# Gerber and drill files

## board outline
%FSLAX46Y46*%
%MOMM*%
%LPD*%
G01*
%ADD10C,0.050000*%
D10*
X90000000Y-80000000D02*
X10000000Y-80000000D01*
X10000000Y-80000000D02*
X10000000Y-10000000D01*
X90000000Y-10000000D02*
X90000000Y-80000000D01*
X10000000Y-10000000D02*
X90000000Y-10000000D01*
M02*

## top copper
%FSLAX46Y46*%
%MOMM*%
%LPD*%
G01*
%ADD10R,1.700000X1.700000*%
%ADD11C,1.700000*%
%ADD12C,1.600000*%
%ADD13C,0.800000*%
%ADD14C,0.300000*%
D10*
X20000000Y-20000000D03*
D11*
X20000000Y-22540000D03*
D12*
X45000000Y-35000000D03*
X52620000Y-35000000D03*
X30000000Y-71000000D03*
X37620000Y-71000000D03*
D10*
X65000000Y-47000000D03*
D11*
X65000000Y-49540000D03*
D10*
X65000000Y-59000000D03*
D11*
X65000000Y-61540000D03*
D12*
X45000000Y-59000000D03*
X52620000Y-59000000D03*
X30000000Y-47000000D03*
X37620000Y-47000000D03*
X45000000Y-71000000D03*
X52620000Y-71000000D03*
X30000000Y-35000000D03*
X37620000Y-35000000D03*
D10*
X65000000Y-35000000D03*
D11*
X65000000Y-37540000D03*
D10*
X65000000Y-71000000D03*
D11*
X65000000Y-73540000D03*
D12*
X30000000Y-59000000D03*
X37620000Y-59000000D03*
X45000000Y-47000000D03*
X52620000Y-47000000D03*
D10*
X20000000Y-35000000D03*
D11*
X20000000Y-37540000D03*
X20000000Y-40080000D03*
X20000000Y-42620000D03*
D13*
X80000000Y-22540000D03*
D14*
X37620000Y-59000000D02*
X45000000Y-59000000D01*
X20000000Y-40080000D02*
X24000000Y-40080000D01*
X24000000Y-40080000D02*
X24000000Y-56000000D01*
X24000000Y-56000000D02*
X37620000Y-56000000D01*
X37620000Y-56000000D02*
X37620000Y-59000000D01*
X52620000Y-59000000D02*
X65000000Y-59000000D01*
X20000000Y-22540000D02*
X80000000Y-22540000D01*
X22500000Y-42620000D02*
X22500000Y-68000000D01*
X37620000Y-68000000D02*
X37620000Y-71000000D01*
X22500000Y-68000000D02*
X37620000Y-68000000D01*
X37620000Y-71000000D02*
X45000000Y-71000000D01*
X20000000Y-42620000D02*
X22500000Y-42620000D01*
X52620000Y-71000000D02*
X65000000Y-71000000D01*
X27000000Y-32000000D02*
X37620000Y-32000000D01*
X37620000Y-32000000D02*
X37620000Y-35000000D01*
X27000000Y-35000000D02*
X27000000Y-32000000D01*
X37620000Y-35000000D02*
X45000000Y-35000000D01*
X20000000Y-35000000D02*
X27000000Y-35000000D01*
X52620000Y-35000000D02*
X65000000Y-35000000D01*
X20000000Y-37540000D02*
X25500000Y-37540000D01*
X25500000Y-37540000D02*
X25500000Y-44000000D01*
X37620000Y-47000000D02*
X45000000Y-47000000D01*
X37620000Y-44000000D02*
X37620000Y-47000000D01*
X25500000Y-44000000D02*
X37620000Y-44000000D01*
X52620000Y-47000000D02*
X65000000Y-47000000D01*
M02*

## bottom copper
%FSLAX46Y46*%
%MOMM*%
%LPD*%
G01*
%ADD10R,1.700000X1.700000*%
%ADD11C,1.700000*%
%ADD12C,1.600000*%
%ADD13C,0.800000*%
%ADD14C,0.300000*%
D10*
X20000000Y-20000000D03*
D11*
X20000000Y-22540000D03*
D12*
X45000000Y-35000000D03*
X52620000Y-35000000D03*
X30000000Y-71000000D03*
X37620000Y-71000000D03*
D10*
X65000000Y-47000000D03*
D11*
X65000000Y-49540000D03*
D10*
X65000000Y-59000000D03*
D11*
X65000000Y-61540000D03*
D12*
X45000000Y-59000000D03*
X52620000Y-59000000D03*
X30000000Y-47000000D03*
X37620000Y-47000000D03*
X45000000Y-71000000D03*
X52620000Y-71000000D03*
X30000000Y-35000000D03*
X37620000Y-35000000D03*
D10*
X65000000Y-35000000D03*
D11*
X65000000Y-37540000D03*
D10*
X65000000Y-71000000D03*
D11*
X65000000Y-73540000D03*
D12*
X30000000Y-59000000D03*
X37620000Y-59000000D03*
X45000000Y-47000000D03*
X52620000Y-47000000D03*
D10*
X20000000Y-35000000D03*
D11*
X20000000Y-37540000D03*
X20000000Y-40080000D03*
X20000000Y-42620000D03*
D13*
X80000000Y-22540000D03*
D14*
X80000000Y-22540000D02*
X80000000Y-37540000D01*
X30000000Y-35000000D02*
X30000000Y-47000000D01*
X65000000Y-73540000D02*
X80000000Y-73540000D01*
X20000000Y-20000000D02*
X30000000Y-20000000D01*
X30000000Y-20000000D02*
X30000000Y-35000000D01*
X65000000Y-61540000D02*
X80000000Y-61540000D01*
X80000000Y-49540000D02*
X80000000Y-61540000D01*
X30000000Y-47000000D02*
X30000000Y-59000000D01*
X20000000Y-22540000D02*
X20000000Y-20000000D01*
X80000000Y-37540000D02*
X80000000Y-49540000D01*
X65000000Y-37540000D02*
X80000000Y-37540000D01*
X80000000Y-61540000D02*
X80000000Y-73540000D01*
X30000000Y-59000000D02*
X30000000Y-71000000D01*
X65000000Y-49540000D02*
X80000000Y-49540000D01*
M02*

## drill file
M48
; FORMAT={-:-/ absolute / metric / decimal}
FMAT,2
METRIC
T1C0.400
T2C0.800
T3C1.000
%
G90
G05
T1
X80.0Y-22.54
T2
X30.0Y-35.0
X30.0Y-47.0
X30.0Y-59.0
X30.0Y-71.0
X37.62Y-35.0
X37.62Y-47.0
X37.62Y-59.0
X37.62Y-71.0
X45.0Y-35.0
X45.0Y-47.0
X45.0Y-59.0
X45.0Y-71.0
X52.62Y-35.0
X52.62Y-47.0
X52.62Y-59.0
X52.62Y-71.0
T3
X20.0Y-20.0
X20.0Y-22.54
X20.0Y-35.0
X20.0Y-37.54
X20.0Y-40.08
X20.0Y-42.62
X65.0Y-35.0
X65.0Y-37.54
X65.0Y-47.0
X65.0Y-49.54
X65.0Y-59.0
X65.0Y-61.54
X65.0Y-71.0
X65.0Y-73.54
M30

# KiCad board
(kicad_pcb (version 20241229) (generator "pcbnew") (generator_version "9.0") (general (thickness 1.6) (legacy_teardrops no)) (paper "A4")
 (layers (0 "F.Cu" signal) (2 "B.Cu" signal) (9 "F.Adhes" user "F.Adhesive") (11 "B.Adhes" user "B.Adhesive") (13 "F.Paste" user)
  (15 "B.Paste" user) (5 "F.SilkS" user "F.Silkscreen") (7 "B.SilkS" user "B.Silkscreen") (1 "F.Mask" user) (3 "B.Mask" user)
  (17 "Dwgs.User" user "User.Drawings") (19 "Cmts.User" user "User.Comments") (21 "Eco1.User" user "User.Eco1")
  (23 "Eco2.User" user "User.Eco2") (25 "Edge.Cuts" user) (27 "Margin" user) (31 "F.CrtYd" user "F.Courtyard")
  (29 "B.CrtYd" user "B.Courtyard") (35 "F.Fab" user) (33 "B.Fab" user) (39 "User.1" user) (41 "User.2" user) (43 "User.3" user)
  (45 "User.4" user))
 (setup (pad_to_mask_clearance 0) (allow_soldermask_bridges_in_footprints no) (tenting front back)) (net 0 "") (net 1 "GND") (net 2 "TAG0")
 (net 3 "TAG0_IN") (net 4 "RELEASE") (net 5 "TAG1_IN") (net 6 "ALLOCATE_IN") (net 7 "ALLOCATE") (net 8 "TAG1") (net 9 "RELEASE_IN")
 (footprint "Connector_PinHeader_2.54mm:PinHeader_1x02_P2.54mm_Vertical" (layer "F.Cu") (at 20 20)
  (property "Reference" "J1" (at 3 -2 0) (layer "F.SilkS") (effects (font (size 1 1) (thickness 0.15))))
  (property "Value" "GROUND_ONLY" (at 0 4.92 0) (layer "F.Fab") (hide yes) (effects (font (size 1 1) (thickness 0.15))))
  (pad "1" thru_hole rect (at 0 0) (size 1.7 1.7) (drill 1) (layers "*.Cu" "*.Mask") (remove_unused_layers no) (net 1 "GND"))
  (pad "2" thru_hole circle (at 0 2.54) (size 1.7 1.7) (drill 1) (layers "*.Cu" "*.Mask") (remove_unused_layers no) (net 1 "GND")))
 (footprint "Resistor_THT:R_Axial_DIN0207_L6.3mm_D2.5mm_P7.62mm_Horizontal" (layer "F.Cu") (at 45 35)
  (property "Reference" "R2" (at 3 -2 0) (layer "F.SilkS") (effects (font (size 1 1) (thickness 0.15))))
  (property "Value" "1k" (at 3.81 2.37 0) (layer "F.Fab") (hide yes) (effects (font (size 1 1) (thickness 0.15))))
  (pad "1" thru_hole circle (at 0 0) (size 1.6 1.6) (drill 0.8) (layers "*.Cu" "*.Mask") (remove_unused_layers no) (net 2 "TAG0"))
  (pad "2" thru_hole circle (at 7.62 0) (size 1.6 1.6) (drill 0.8) (layers "*.Cu" "*.Mask") (remove_unused_layers no) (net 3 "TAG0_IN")))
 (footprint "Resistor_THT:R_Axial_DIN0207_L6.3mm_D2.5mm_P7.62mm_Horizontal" (layer "F.Cu") (at 30 71)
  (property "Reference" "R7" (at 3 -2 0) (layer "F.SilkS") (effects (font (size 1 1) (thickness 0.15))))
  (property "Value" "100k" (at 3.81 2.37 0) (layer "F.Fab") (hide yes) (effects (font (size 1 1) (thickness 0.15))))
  (pad "1" thru_hole circle (at 0 0) (size 1.6 1.6) (drill 0.8) (layers "*.Cu" "*.Mask") (remove_unused_layers no) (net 1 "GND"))
  (pad "2" thru_hole circle (at 7.62 0) (size 1.6 1.6) (drill 0.8) (layers "*.Cu" "*.Mask") (remove_unused_layers no) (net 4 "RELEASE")))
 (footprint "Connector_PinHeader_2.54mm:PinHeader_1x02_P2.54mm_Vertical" (layer "F.Cu") (at 65 47)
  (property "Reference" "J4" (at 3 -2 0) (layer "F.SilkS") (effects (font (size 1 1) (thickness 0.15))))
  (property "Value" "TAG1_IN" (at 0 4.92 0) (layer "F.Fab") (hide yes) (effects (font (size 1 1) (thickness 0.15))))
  (pad "1" thru_hole rect (at 0 0) (size 1.7 1.7) (drill 1) (layers "*.Cu" "*.Mask") (remove_unused_layers no) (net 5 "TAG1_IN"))
  (pad "2" thru_hole circle (at 0 2.54) (size 1.7 1.7) (drill 1) (layers "*.Cu" "*.Mask") (remove_unused_layers no) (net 1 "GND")))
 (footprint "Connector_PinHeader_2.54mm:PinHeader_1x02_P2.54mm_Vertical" (layer "F.Cu") (at 65 59)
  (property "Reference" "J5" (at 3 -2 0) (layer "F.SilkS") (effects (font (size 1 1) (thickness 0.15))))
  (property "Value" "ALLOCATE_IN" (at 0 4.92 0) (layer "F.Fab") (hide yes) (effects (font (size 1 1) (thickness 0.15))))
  (pad "1" thru_hole rect (at 0 0) (size 1.7 1.7) (drill 1) (layers "*.Cu" "*.Mask") (remove_unused_layers no) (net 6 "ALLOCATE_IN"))
  (pad "2" thru_hole circle (at 0 2.54) (size 1.7 1.7) (drill 1) (layers "*.Cu" "*.Mask") (remove_unused_layers no) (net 1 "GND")))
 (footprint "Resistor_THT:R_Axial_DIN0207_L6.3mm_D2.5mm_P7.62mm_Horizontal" (layer "F.Cu") (at 45 59)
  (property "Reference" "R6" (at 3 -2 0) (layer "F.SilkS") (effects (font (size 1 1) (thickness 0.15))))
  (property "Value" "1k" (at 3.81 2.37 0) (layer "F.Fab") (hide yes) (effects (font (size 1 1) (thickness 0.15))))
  (pad "1" thru_hole circle (at 0 0) (size 1.6 1.6) (drill 0.8) (layers "*.Cu" "*.Mask") (remove_unused_layers no) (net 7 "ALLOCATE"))
  (pad "2" thru_hole circle (at 7.62 0) (size 1.6 1.6) (drill 0.8) (layers "*.Cu" "*.Mask") (remove_unused_layers no) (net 6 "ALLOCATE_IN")))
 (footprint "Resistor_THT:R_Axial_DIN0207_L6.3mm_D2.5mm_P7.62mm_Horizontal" (layer "F.Cu") (at 30 47)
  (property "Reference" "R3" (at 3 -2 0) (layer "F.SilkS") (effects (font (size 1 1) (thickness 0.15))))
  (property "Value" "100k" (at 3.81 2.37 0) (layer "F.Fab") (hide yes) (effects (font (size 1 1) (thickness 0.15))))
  (pad "1" thru_hole circle (at 0 0) (size 1.6 1.6) (drill 0.8) (layers "*.Cu" "*.Mask") (remove_unused_layers no) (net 1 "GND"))
  (pad "2" thru_hole circle (at 7.62 0) (size 1.6 1.6) (drill 0.8) (layers "*.Cu" "*.Mask") (remove_unused_layers no) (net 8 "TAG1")))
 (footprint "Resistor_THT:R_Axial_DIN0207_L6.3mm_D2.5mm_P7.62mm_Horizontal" (layer "F.Cu") (at 45 71)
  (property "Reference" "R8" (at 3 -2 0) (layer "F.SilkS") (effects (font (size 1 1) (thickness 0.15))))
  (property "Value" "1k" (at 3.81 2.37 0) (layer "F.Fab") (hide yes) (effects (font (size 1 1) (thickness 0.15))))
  (pad "1" thru_hole circle (at 0 0) (size 1.6 1.6) (drill 0.8) (layers "*.Cu" "*.Mask") (remove_unused_layers no) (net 4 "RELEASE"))
  (pad "2" thru_hole circle (at 7.62 0) (size 1.6 1.6) (drill 0.8) (layers "*.Cu" "*.Mask") (remove_unused_layers no) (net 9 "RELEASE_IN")))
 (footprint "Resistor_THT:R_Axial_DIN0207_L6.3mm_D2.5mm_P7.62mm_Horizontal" (layer "F.Cu") (at 30 35)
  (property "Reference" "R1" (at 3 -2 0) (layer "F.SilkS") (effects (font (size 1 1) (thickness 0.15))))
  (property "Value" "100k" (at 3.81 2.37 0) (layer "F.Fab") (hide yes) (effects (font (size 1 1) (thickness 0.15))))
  (pad "1" thru_hole circle (at 0 0) (size 1.6 1.6) (drill 0.8) (layers "*.Cu" "*.Mask") (remove_unused_layers no) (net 1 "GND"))
  (pad "2" thru_hole circle (at 7.62 0) (size 1.6 1.6) (drill 0.8) (layers "*.Cu" "*.Mask") (remove_unused_layers no) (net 2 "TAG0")))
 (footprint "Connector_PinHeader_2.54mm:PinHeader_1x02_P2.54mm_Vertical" (layer "F.Cu") (at 65 35)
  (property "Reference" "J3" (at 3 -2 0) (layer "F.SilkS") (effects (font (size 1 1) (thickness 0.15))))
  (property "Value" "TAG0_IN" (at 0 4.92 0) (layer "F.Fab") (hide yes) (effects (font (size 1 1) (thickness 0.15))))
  (pad "1" thru_hole rect (at 0 0) (size 1.7 1.7) (drill 1) (layers "*.Cu" "*.Mask") (remove_unused_layers no) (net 3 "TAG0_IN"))
  (pad "2" thru_hole circle (at 0 2.54) (size 1.7 1.7) (drill 1) (layers "*.Cu" "*.Mask") (remove_unused_layers no) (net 1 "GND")))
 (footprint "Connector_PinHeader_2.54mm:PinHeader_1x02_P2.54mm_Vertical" (layer "F.Cu") (at 65 71)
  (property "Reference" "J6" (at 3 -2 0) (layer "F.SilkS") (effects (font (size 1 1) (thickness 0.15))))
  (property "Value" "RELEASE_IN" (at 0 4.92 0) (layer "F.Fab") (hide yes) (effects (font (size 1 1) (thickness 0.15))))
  (pad "1" thru_hole rect (at 0 0) (size 1.7 1.7) (drill 1) (layers "*.Cu" "*.Mask") (remove_unused_layers no) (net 9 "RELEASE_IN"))
  (pad "2" thru_hole circle (at 0 2.54) (size 1.7 1.7) (drill 1) (layers "*.Cu" "*.Mask") (remove_unused_layers no) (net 1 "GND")))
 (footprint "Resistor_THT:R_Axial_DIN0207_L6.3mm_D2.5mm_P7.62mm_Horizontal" (layer "F.Cu") (at 30 59)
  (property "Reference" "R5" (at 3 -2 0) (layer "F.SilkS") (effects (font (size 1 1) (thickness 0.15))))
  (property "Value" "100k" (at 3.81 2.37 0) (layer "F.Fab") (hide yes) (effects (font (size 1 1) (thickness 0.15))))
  (pad "1" thru_hole circle (at 0 0) (size 1.6 1.6) (drill 0.8) (layers "*.Cu" "*.Mask") (remove_unused_layers no) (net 1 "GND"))
  (pad "2" thru_hole circle (at 7.62 0) (size 1.6 1.6) (drill 0.8) (layers "*.Cu" "*.Mask") (remove_unused_layers no) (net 7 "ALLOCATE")))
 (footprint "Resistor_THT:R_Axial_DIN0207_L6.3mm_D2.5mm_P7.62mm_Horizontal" (layer "F.Cu") (at 45 47)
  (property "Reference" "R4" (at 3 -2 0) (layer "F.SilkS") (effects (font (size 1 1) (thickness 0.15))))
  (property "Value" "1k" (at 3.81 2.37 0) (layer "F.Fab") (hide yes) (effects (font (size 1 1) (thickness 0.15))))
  (pad "1" thru_hole circle (at 0 0) (size 1.6 1.6) (drill 0.8) (layers "*.Cu" "*.Mask") (remove_unused_layers no) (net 8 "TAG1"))
  (pad "2" thru_hole circle (at 7.62 0) (size 1.6 1.6) (drill 0.8) (layers "*.Cu" "*.Mask") (remove_unused_layers no) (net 5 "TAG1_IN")))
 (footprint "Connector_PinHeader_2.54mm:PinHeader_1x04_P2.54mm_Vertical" (layer "F.Cu") (at 20 35)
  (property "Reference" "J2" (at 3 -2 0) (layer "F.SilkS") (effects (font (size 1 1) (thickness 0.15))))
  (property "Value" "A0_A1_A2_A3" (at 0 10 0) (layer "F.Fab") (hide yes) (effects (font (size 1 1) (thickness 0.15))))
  (pad "1" thru_hole rect (at 0 0) (size 1.7 1.7) (drill 1) (layers "*.Cu" "*.Mask") (remove_unused_layers no) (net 2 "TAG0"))
  (pad "2" thru_hole circle (at 0 2.54) (size 1.7 1.7) (drill 1) (layers "*.Cu" "*.Mask") (remove_unused_layers no) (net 8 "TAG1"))
  (pad "3" thru_hole circle (at 0 5.08) (size 1.7 1.7) (drill 1) (layers "*.Cu" "*.Mask") (remove_unused_layers no) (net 7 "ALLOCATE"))
  (pad "4" thru_hole circle (at 0 7.62) (size 1.7 1.7) (drill 1) (layers "*.Cu" "*.Mask") (remove_unused_layers no) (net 4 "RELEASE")))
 (gr_line (start 90 80) (end 10 80) (stroke (width 0.05) (type default)) (layer "Edge.Cuts"))
 (gr_line (start 10 80) (end 10 10) (stroke (width 0.05) (type default)) (layer "Edge.Cuts"))
 (gr_line (start 90 10) (end 90 80) (stroke (width 0.05) (type default)) (layer "Edge.Cuts"))
 (gr_line (start 10 10) (end 90 10) (stroke (width 0.05) (type default)) (layer "Edge.Cuts"))
 (segment (start 37.62 59) (end 45 59) (width 0.3) (layer "F.Cu") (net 7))
 (segment (start 20 40.08) (end 24 40.08) (width 0.3) (layer "F.Cu") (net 7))
 (segment (start 24 40.08) (end 24 56) (width 0.3) (layer "F.Cu") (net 7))
 (segment (start 24 56) (end 37.62 56) (width 0.3) (layer "F.Cu") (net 7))
 (segment (start 37.62 56) (end 37.62 59) (width 0.3) (layer "F.Cu") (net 7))
 (segment (start 52.62 59) (end 65 59) (width 0.3) (layer "F.Cu") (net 6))
 (segment (start 20 22.54) (end 80 22.54) (width 0.3) (layer "F.Cu") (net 1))
 (via (at 80 22.54) (size 0.8) (drill 0.4) (layers "F.Cu" "B.Cu") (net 1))
 (segment (start 80 22.54) (end 80 37.54) (width 0.3) (layer "B.Cu") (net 1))
 (segment (start 30 35) (end 30 47) (width 0.3) (layer "B.Cu") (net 1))
 (segment (start 65 73.54) (end 80 73.54) (width 0.3) (layer "B.Cu") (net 1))
 (segment (start 20 20) (end 30 20) (width 0.3) (layer "B.Cu") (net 1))
 (segment (start 30 20) (end 30 35) (width 0.3) (layer "B.Cu") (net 1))
 (segment (start 65 61.54) (end 80 61.54) (width 0.3) (layer "B.Cu") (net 1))
 (segment (start 80 49.54) (end 80 61.54) (width 0.3) (layer "B.Cu") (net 1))
 (segment (start 30 47) (end 30 59) (width 0.3) (layer "B.Cu") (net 1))
 (segment (start 20 22.54) (end 20 20) (width 0.3) (layer "B.Cu") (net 1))
 (segment (start 80 37.54) (end 80 49.54) (width 0.3) (layer "B.Cu") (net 1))
 (segment (start 65 37.54) (end 80 37.54) (width 0.3) (layer "B.Cu") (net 1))
 (segment (start 80 61.54) (end 80 73.54) (width 0.3) (layer "B.Cu") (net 1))
 (segment (start 30 59) (end 30 71) (width 0.3) (layer "B.Cu") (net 1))
 (segment (start 65 49.54) (end 80 49.54) (width 0.3) (layer "B.Cu") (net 1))
 (segment (start 22.5 42.62) (end 22.5 68) (width 0.3) (layer "F.Cu") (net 4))
 (segment (start 37.62 68) (end 37.62 71) (width 0.3) (layer "F.Cu") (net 4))
 (segment (start 22.5 68) (end 37.62 68) (width 0.3) (layer "F.Cu") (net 4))
 (segment (start 37.62 71) (end 45 71) (width 0.3) (layer "F.Cu") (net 4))
 (segment (start 20 42.62) (end 22.5 42.62) (width 0.3) (layer "F.Cu") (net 4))
 (segment (start 52.62 71) (end 65 71) (width 0.3) (layer "F.Cu") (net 9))
 (segment (start 27 32) (end 37.62 32) (width 0.3) (layer "F.Cu") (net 2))
 (segment (start 37.62 32) (end 37.62 35) (width 0.3) (layer "F.Cu") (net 2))
 (segment (start 27 35) (end 27 32) (width 0.3) (layer "F.Cu") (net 2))
 (segment (start 37.62 35) (end 45 35) (width 0.3) (layer "F.Cu") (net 2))
 (segment (start 20 35) (end 27 35) (width 0.3) (layer "F.Cu") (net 2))
 (segment (start 52.62 35) (end 65 35) (width 0.3) (layer "F.Cu") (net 3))
 (segment (start 20 37.54) (end 25.5 37.54) (width 0.3) (layer "F.Cu") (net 8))
 (segment (start 25.5 37.54) (end 25.5 44) (width 0.3) (layer "F.Cu") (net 8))
 (segment (start 37.62 47) (end 45 47) (width 0.3) (layer "F.Cu") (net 8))
 (segment (start 37.62 44) (end 37.62 47) (width 0.3) (layer "F.Cu") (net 8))
 (segment (start 25.5 44) (end 37.62 44) (width 0.3) (layer "F.Cu") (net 8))
 (segment (start 52.62 47) (end 65 47) (width 0.3) (layer "F.Cu") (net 5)))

